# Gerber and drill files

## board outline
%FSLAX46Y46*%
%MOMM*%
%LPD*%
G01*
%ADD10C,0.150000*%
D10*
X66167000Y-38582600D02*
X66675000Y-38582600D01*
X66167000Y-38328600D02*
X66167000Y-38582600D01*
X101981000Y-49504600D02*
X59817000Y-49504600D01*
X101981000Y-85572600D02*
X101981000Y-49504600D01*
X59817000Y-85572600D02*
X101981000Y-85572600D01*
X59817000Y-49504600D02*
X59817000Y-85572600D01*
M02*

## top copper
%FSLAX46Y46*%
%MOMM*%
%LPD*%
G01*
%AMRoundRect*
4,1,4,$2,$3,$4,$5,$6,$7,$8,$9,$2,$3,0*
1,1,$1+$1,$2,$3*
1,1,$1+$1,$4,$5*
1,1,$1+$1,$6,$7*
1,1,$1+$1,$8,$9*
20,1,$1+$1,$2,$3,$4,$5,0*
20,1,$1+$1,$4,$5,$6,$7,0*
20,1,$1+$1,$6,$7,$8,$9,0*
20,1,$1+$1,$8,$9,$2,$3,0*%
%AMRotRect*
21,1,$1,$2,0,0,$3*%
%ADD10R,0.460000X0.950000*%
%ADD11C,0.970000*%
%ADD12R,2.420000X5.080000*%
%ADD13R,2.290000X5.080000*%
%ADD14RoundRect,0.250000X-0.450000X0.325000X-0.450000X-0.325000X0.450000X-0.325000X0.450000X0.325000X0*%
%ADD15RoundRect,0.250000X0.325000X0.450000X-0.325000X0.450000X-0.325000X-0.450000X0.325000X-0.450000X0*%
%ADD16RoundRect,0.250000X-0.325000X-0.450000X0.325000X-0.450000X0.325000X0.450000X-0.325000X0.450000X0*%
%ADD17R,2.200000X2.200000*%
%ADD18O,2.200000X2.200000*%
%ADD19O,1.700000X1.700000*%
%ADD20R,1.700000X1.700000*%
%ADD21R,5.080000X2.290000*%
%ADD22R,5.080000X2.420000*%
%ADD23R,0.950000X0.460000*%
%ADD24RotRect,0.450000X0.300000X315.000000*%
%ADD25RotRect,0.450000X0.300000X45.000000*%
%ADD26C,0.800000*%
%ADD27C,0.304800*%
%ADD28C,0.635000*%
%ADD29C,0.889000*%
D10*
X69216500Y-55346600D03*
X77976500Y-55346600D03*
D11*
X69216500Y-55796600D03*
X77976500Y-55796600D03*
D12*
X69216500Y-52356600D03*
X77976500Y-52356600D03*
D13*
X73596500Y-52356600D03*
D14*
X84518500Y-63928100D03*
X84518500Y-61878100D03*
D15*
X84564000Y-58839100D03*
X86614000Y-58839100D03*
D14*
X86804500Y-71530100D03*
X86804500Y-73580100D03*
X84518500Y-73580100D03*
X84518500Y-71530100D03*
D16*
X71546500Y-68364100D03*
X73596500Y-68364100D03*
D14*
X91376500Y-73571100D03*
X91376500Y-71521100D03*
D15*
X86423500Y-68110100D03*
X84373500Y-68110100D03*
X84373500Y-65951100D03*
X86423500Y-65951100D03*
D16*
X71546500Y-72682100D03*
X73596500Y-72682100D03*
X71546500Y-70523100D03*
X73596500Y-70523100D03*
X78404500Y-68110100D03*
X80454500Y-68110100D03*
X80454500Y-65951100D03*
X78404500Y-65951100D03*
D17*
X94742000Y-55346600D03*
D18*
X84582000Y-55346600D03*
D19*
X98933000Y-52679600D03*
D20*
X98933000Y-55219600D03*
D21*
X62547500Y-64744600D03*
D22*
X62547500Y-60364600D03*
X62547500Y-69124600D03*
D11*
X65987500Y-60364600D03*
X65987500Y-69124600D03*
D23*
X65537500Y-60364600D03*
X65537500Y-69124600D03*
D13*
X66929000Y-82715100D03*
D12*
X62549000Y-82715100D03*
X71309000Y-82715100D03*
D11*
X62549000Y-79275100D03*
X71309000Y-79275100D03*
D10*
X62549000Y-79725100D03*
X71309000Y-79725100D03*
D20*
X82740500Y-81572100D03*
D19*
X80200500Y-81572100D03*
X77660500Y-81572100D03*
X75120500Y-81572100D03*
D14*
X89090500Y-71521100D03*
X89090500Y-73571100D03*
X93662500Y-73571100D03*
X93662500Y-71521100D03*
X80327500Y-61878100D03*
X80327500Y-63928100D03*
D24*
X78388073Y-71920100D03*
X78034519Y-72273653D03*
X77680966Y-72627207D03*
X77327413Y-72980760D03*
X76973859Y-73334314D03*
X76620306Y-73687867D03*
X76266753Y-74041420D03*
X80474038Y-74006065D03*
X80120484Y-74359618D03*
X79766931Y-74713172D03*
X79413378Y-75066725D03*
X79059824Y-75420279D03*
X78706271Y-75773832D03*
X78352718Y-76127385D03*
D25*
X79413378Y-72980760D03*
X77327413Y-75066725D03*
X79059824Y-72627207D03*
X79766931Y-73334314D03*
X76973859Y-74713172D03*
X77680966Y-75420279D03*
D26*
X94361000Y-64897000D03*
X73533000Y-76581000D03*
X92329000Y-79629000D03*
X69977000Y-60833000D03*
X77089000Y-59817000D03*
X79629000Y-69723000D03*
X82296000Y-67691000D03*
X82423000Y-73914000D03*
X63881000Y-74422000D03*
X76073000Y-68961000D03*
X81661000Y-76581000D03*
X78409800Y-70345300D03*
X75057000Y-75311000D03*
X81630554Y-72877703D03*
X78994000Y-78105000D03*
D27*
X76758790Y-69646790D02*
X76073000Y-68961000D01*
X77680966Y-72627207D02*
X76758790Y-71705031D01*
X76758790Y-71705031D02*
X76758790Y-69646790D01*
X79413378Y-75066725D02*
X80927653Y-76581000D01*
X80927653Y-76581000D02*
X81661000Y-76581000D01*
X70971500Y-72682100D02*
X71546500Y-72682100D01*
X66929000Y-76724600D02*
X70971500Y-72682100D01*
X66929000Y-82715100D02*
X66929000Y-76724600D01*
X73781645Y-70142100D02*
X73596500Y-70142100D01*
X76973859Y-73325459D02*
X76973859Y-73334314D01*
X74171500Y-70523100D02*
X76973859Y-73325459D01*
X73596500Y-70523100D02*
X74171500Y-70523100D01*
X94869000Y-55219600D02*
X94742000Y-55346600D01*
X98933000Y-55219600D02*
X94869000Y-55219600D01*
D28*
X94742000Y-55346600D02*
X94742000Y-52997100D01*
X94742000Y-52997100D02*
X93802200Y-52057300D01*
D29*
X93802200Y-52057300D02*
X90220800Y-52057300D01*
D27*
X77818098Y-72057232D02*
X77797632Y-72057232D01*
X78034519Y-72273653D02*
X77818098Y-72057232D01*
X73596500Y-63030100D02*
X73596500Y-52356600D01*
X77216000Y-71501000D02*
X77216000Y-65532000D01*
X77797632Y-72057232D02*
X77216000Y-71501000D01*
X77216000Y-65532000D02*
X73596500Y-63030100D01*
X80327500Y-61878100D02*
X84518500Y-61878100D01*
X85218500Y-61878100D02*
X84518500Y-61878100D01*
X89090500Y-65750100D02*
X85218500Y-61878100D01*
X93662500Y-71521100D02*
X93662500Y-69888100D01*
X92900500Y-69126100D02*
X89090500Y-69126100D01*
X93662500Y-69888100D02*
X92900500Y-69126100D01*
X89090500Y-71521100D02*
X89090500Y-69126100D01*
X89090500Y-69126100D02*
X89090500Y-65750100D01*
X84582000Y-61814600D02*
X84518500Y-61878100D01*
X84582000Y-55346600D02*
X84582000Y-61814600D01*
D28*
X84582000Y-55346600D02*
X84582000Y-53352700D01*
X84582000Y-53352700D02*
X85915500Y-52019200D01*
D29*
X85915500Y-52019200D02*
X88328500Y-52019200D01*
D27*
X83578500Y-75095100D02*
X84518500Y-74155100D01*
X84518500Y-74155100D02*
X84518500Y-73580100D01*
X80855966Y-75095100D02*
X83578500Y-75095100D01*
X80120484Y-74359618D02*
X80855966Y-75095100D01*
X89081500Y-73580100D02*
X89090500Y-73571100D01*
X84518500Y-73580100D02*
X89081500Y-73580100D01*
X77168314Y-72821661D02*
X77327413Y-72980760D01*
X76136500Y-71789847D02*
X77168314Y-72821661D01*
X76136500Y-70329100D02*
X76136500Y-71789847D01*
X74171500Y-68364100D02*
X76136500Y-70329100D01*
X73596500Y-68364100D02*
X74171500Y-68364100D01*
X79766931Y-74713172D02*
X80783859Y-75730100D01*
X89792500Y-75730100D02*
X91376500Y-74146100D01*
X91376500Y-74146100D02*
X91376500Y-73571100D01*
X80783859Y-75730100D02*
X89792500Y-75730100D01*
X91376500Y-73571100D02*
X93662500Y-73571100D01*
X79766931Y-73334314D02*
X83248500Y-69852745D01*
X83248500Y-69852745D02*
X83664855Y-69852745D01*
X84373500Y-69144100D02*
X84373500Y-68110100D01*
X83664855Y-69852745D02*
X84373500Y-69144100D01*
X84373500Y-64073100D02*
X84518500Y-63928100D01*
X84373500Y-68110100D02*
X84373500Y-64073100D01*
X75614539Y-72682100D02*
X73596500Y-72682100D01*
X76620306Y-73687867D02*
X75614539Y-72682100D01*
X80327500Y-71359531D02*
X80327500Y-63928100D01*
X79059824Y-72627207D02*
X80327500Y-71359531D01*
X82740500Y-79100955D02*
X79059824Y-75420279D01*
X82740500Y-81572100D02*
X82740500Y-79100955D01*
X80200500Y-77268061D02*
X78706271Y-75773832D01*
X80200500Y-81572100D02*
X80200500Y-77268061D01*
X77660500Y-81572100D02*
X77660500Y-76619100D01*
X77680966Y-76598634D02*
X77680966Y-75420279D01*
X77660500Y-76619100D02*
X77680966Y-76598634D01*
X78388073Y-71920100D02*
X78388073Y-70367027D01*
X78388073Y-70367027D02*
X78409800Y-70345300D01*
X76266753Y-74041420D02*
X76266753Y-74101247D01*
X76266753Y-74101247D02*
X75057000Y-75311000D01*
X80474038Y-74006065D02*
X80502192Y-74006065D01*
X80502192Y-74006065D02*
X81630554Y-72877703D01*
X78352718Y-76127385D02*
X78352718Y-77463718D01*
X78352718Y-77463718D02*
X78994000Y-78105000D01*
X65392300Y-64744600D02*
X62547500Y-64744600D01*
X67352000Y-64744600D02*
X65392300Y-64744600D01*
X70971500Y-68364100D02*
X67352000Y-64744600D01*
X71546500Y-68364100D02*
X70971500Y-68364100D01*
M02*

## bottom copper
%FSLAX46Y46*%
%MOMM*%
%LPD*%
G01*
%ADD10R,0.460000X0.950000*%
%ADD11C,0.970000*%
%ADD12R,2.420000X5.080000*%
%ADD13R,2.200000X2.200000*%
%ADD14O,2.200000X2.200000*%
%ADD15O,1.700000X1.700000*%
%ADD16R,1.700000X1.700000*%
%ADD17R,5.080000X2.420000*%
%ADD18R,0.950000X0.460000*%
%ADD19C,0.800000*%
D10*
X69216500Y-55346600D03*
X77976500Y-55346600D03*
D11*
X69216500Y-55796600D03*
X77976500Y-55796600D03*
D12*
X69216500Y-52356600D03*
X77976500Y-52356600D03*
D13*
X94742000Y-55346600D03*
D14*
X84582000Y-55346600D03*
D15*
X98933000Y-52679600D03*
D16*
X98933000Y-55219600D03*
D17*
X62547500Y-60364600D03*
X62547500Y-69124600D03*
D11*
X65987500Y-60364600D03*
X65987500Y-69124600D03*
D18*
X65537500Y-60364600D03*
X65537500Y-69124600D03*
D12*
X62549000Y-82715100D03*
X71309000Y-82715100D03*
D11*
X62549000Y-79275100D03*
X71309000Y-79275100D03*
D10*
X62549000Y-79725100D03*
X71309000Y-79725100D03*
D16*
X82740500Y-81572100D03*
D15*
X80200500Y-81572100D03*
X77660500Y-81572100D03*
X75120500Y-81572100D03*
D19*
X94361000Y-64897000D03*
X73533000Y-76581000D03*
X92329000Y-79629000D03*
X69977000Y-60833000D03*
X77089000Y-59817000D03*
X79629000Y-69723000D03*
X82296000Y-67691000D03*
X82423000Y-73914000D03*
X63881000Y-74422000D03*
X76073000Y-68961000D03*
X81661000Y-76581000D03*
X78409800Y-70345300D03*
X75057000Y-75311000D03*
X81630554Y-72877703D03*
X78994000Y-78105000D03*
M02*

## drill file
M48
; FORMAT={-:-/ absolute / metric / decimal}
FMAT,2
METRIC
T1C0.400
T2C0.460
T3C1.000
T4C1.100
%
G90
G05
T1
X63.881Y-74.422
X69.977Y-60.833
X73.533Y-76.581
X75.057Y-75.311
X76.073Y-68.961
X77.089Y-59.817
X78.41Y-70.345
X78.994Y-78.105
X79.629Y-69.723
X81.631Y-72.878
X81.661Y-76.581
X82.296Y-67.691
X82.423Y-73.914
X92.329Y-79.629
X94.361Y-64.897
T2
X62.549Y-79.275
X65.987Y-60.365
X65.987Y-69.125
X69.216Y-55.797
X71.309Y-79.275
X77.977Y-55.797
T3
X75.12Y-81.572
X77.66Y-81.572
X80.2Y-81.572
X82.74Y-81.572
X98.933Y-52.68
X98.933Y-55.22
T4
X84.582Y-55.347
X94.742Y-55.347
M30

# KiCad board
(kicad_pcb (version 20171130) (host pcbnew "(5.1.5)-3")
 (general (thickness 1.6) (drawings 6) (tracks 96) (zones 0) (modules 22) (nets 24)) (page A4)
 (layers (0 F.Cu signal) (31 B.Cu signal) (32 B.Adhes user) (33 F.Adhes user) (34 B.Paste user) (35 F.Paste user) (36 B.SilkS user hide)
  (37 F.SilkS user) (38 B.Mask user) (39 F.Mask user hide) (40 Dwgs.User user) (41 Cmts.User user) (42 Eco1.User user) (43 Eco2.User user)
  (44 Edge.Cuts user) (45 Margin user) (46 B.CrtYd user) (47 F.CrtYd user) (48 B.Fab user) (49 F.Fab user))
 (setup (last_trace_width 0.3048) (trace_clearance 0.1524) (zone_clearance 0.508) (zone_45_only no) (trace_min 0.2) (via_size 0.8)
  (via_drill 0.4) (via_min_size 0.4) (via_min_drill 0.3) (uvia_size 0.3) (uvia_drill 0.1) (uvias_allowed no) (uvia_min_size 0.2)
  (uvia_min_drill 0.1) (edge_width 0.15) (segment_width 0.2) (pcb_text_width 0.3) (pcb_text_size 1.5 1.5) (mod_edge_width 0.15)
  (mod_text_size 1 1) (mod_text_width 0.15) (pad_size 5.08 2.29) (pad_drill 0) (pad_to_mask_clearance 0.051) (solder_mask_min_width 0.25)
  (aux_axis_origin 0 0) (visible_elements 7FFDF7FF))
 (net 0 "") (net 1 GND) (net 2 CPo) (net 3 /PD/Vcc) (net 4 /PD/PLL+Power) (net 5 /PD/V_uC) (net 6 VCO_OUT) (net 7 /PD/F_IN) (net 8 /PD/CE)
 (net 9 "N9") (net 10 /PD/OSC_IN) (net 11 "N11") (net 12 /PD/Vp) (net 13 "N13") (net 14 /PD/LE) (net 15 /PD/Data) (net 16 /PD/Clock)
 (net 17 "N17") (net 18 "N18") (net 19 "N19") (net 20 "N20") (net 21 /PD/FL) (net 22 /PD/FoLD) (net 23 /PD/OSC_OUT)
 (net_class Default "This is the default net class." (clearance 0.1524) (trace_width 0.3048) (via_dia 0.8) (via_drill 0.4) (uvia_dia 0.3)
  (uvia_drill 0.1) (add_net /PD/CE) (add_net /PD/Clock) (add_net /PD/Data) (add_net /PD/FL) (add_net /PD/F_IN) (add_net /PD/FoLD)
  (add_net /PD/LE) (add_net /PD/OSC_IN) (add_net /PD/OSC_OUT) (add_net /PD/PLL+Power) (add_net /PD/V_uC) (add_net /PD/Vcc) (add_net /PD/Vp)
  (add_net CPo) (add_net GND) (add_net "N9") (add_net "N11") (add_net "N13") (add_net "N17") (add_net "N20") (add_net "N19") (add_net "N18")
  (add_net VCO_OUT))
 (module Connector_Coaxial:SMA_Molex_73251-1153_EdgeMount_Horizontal (layer F.Cu) (at 73.5965 54.0766 270)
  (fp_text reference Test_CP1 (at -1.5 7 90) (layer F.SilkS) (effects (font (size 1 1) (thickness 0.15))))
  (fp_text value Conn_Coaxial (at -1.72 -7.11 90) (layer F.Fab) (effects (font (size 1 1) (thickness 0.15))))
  (pad 2 smd rect (at 1.27 4.38 270) (size 0.95 0.46) (layers B.Cu) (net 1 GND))
  (pad 2 smd rect (at 1.27 -4.38 270) (size 0.95 0.46) (layers B.Cu) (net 1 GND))
  (pad 2 smd rect (at 1.27 4.38 270) (size 0.95 0.46) (layers F.Cu) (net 1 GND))
  (pad 2 smd rect (at 1.27 -4.38 270) (size 0.95 0.46) (layers F.Cu) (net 1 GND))
  (pad 2 thru_hole circle (at 1.72 4.38 270) (size 0.97 0.97) (drill 0.46) (layers *.Cu) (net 1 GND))
  (pad 2 thru_hole circle (at 1.72 -4.38 270) (size 0.97 0.97) (drill 0.46) (layers *.Cu) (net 1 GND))
  (pad 2 smd rect (at -1.72 4.38 270) (size 5.08 2.42) (layers B.Cu B.Paste B.Mask) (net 1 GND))
  (pad 2 smd rect (at -1.72 -4.38 270) (size 5.08 2.42) (layers B.Cu B.Paste B.Mask) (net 1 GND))
  (pad 2 smd rect (at -1.72 4.38 270) (size 5.08 2.42) (layers F.Cu F.Paste F.Mask) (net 1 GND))
  (pad 2 smd rect (at -1.72 -4.38 270) (size 5.08 2.42) (layers F.Cu F.Paste F.Mask) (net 1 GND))
  (pad 1 smd rect (at -1.72 0 270) (size 5.08 2.29) (layers F.Cu F.Paste F.Mask) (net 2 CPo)))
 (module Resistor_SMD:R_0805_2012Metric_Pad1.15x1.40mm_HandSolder (layer F.Cu) (at 84.5185 62.9031 270)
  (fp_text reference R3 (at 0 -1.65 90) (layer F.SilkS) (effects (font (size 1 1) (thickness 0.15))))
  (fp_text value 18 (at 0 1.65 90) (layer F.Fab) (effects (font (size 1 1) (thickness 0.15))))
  (pad 2 smd roundrect (at 1.025 0 270) (size 1.15 1.4) (layers F.Cu F.Paste F.Mask) (roundrect_rratio 0.217391) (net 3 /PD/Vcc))
  (pad 1 smd roundrect (at -1.025 0 270) (size 1.15 1.4) (layers F.Cu F.Paste F.Mask) (roundrect_rratio 0.217391) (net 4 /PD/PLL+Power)))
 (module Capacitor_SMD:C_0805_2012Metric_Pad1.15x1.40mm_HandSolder (layer F.Cu) (at 85.589 58.8391 180)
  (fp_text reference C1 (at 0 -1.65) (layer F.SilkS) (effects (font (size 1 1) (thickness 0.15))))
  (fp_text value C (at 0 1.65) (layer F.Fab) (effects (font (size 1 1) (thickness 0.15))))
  (pad 2 smd roundrect (at 1.025 0 180) (size 1.15 1.4) (layers F.Cu F.Paste F.Mask) (roundrect_rratio 0.217391) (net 4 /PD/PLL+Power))
  (pad 1 smd roundrect (at -1.025 0 180) (size 1.15 1.4) (layers F.Cu F.Paste F.Mask) (roundrect_rratio 0.217391) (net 1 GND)))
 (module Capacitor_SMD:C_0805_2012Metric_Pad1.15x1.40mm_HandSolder (layer F.Cu) (at 86.8045 72.5551 270)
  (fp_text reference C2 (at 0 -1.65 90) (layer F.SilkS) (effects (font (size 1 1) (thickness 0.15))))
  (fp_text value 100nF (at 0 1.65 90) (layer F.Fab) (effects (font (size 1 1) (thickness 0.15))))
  (pad 1 smd roundrect (at -1.025 0 270) (size 1.15 1.4) (layers F.Cu F.Paste F.Mask) (roundrect_rratio 0.217391) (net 1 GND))
  (pad 2 smd roundrect (at 1.025 0 270) (size 1.15 1.4) (layers F.Cu F.Paste F.Mask) (roundrect_rratio 0.217391) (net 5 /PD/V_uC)))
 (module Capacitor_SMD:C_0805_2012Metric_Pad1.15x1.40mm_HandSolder (layer F.Cu) (at 84.5185 72.5551 270)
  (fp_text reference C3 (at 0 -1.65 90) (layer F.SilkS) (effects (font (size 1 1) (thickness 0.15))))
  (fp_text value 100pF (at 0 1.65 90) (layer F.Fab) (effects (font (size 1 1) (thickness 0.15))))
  (pad 2 smd roundrect (at 1.025 0 270) (size 1.15 1.4) (layers F.Cu F.Paste F.Mask) (roundrect_rratio 0.217391) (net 5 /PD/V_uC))
  (pad 1 smd roundrect (at -1.025 0 270) (size 1.15 1.4) (layers F.Cu F.Paste F.Mask) (roundrect_rratio 0.217391) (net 1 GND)))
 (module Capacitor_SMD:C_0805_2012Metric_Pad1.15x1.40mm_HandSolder (layer F.Cu) (at 72.5715 68.3641)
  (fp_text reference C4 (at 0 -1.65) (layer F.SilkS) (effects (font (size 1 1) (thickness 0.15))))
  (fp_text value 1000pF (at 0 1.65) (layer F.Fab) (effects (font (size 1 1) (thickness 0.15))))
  (pad 1 smd roundrect (at -1.025 0) (size 1.15 1.4) (layers F.Cu F.Paste F.Mask) (roundrect_rratio 0.217391) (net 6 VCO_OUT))
  (pad 2 smd roundrect (at 1.025 0) (size 1.15 1.4) (layers F.Cu F.Paste F.Mask) (roundrect_rratio 0.217391) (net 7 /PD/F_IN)))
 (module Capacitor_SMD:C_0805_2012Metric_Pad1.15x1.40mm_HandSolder (layer F.Cu) (at 91.3765 72.5461 270)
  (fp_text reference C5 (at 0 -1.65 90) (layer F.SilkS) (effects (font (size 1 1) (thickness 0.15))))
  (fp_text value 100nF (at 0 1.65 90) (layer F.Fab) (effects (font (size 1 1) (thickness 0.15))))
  (pad 2 smd roundrect (at 1.025 0 270) (size 1.15 1.4) (layers F.Cu F.Paste F.Mask) (roundrect_rratio 0.217391) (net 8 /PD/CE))
  (pad 1 smd roundrect (at -1.025 0 270) (size 1.15 1.4) (layers F.Cu F.Paste F.Mask) (roundrect_rratio 0.217391) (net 1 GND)))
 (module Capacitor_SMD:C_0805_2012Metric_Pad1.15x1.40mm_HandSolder (layer F.Cu) (at 85.3985 68.1101 180)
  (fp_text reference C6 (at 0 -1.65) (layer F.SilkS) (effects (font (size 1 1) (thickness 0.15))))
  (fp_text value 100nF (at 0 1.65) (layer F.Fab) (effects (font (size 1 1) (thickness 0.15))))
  (pad 1 smd roundrect (at -1.025 0 180) (size 1.15 1.4) (layers F.Cu F.Paste F.Mask) (roundrect_rratio 0.217391) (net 1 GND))
  (pad 2 smd roundrect (at 1.025 0 180) (size 1.15 1.4) (layers F.Cu F.Paste F.Mask) (roundrect_rratio 0.217391) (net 3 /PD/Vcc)))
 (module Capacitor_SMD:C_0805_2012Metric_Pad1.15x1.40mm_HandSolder (layer F.Cu) (at 85.3985 65.9511 180)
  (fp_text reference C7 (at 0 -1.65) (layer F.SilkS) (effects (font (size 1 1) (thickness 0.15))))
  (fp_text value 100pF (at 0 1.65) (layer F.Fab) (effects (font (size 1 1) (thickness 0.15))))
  (pad 2 smd roundrect (at 1.025 0 180) (size 1.15 1.4) (layers F.Cu F.Paste F.Mask) (roundrect_rratio 0.217391) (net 3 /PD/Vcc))
  (pad 1 smd roundrect (at -1.025 0 180) (size 1.15 1.4) (layers F.Cu F.Paste F.Mask) (roundrect_rratio 0.217391) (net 1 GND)))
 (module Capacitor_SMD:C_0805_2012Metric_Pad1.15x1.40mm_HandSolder (layer F.Cu) (at 72.5715 72.6821)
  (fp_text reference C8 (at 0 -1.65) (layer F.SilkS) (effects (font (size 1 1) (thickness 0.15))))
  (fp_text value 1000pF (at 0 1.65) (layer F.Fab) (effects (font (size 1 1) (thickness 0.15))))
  (pad 1 smd roundrect (at -1.025 0) (size 1.15 1.4) (layers F.Cu F.Paste F.Mask) (roundrect_rratio 0.217391) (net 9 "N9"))
  (pad 2 smd roundrect (at 1.025 0) (size 1.15 1.4) (layers F.Cu F.Paste F.Mask) (roundrect_rratio 0.217391) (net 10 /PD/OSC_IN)))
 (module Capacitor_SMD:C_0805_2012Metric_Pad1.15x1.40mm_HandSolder (layer F.Cu) (at 72.5715 70.5231)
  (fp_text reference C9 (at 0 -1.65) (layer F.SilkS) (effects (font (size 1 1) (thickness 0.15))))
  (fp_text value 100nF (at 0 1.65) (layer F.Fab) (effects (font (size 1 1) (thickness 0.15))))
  (pad 1 smd roundrect (at -1.025 0) (size 1.15 1.4) (layers F.Cu F.Paste F.Mask) (roundrect_rratio 0.217391) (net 1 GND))
  (pad 2 smd roundrect (at 1.025 0) (size 1.15 1.4) (layers F.Cu F.Paste F.Mask) (roundrect_rratio 0.217391) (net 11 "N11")))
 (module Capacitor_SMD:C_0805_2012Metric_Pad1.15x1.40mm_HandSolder (layer F.Cu) (at 79.4295 68.1101)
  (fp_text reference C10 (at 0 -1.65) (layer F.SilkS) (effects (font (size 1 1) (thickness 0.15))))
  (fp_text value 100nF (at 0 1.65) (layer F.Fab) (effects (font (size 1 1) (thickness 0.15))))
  (pad 1 smd roundrect (at -1.025 0) (size 1.15 1.4) (layers F.Cu F.Paste F.Mask) (roundrect_rratio 0.217391) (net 1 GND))
  (pad 2 smd roundrect (at 1.025 0) (size 1.15 1.4) (layers F.Cu F.Paste F.Mask) (roundrect_rratio 0.217391) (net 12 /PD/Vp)))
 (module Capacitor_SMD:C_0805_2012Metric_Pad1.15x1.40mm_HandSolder (layer F.Cu) (at 79.4295 65.9511)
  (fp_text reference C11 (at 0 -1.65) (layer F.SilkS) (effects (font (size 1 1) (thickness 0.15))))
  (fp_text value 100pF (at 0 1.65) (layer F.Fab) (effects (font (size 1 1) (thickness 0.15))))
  (pad 2 smd roundrect (at 1.025 0) (size 1.15 1.4) (layers F.Cu F.Paste F.Mask) (roundrect_rratio 0.217391) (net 12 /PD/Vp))
  (pad 1 smd roundrect (at -1.025 0) (size 1.15 1.4) (layers F.Cu F.Paste F.Mask) (roundrect_rratio 0.217391) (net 1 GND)))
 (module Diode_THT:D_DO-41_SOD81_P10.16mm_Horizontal (layer F.Cu) (at 94.742 55.3466 180)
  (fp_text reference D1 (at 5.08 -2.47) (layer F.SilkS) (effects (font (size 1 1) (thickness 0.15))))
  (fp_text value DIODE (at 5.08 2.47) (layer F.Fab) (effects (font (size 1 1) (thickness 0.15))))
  (pad 1 thru_hole rect (at 0 0 180) (size 2.2 2.2) (drill 1.1) (layers *.Cu *.Mask) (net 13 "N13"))
  (pad 2 thru_hole oval (at 10.16 0 180) (size 2.2 2.2) (drill 1.1) (layers *.Cu *.Mask) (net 4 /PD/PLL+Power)))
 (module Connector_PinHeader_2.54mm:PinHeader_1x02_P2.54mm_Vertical (layer F.Cu) (at 98.933 55.2196 180)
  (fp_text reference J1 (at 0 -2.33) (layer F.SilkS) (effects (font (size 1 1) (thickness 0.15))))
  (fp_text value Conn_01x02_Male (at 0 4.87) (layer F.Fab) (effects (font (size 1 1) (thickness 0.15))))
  (pad 2 thru_hole oval (at 0 2.54 180) (size 1.7 1.7) (drill 1) (layers *.Cu *.Mask) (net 1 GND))
  (pad 1 thru_hole rect (at 0 0 180) (size 1.7 1.7) (drill 1) (layers *.Cu *.Mask) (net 13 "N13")))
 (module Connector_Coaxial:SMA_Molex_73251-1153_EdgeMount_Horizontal (layer F.Cu) (at 64.2675 64.7446)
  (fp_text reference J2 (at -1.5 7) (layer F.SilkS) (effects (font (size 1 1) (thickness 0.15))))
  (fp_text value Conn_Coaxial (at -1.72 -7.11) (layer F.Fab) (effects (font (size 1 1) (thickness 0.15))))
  (pad 1 smd rect (at -1.72 0) (size 5.08 2.29) (layers F.Cu F.Paste F.Mask) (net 6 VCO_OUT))
  (pad 2 smd rect (at -1.72 -4.38) (size 5.08 2.42) (layers F.Cu F.Paste F.Mask) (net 1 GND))
  (pad 2 smd rect (at -1.72 4.38) (size 5.08 2.42) (layers F.Cu F.Paste F.Mask) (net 1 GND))
  (pad 2 smd rect (at -1.72 -4.38) (size 5.08 2.42) (layers B.Cu B.Paste B.Mask) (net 1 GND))
  (pad 2 smd rect (at -1.72 4.38) (size 5.08 2.42) (layers B.Cu B.Paste B.Mask) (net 1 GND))
  (pad 2 thru_hole circle (at 1.72 -4.38) (size 0.97 0.97) (drill 0.46) (layers *.Cu) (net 1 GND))
  (pad 2 thru_hole circle (at 1.72 4.38) (size 0.97 0.97) (drill 0.46) (layers *.Cu) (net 1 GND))
  (pad 2 smd rect (at 1.27 -4.38) (size 0.95 0.46) (layers F.Cu) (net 1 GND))
  (pad 2 smd rect (at 1.27 4.38) (size 0.95 0.46) (layers F.Cu) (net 1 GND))
  (pad 2 smd rect (at 1.27 -4.38) (size 0.95 0.46) (layers B.Cu) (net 1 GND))
  (pad 2 smd rect (at 1.27 4.38) (size 0.95 0.46) (layers B.Cu) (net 1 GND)))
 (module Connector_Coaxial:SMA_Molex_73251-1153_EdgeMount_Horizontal (layer F.Cu) (at 66.929 80.9951 90)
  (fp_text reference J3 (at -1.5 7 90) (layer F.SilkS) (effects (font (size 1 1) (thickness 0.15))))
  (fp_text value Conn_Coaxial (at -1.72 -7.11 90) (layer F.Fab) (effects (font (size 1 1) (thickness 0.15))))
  (pad 1 smd rect (at -1.72 0 90) (size 5.08 2.29) (layers F.Cu F.Paste F.Mask) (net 9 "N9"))
  (pad 2 smd rect (at -1.72 -4.38 90) (size 5.08 2.42) (layers F.Cu F.Paste F.Mask) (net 1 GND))
  (pad 2 smd rect (at -1.72 4.38 90) (size 5.08 2.42) (layers F.Cu F.Paste F.Mask) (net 1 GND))
  (pad 2 smd rect (at -1.72 -4.38 90) (size 5.08 2.42) (layers B.Cu B.Paste B.Mask) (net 1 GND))
  (pad 2 smd rect (at -1.72 4.38 90) (size 5.08 2.42) (layers B.Cu B.Paste B.Mask) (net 1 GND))
  (pad 2 thru_hole circle (at 1.72 -4.38 90) (size 0.97 0.97) (drill 0.46) (layers *.Cu) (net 1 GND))
  (pad 2 thru_hole circle (at 1.72 4.38 90) (size 0.97 0.97) (drill 0.46) (layers *.Cu) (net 1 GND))
  (pad 2 smd rect (at 1.27 -4.38 90) (size 0.95 0.46) (layers F.Cu) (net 1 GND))
  (pad 2 smd rect (at 1.27 4.38 90) (size 0.95 0.46) (layers F.Cu) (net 1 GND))
  (pad 2 smd rect (at 1.27 -4.38 90) (size 0.95 0.46) (layers B.Cu) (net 1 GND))
  (pad 2 smd rect (at 1.27 4.38 90) (size 0.95 0.46) (layers B.Cu) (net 1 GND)))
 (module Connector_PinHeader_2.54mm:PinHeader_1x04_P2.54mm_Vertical (layer F.Cu) (at 82.7405 81.5721 270)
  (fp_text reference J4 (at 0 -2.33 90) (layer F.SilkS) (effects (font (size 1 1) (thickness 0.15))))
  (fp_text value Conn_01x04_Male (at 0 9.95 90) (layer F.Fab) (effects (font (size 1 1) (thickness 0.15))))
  (pad 1 thru_hole rect (at 0 0 270) (size 1.7 1.7) (drill 1) (layers *.Cu *.Mask) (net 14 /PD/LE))
  (pad 2 thru_hole oval (at 0 2.54 270) (size 1.7 1.7) (drill 1) (layers *.Cu *.Mask) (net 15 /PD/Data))
  (pad 3 thru_hole oval (at 0 5.08 270) (size 1.7 1.7) (drill 1) (layers *.Cu *.Mask) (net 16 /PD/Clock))
  (pad 4 thru_hole oval (at 0 7.62 270) (size 1.7 1.7) (drill 1) (layers *.Cu *.Mask) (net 1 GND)))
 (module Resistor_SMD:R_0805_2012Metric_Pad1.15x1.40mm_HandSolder (layer F.Cu) (at 89.0905 72.5461 270)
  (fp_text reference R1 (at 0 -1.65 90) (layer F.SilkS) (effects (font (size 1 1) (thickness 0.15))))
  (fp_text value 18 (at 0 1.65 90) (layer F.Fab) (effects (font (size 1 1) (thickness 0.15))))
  (pad 1 smd roundrect (at -1.025 0 270) (size 1.15 1.4) (layers F.Cu F.Paste F.Mask) (roundrect_rratio 0.217391) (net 4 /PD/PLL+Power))
  (pad 2 smd roundrect (at 1.025 0 270) (size 1.15 1.4) (layers F.Cu F.Paste F.Mask) (roundrect_rratio 0.217391) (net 5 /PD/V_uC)))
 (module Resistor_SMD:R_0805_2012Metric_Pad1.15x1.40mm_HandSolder (layer F.Cu) (at 93.6625 72.5461 270)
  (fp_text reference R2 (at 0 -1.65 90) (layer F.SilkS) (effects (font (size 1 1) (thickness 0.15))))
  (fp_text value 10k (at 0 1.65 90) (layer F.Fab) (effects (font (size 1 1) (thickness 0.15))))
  (pad 2 smd roundrect (at 1.025 0 270) (size 1.15 1.4) (layers F.Cu F.Paste F.Mask) (roundrect_rratio 0.217391) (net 8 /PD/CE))
  (pad 1 smd roundrect (at -1.025 0 270) (size 1.15 1.4) (layers F.Cu F.Paste F.Mask) (roundrect_rratio 0.217391) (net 4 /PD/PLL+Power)))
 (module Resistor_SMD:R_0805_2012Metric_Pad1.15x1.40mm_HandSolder (layer F.Cu) (at 80.3275 62.9031 270)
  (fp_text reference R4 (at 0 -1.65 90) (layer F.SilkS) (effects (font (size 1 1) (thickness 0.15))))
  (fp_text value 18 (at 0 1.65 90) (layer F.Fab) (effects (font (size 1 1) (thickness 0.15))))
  (pad 1 smd roundrect (at -1.025 0 270) (size 1.15 1.4) (layers F.Cu F.Paste F.Mask) (roundrect_rratio 0.217391) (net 4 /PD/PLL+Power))
  (pad 2 smd roundrect (at 1.025 0 270) (size 1.15 1.4) (layers F.Cu F.Paste F.Mask) (roundrect_rratio 0.217391) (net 12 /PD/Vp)))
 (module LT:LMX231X (layer F.Cu) (at 81.2165 71.9201 315)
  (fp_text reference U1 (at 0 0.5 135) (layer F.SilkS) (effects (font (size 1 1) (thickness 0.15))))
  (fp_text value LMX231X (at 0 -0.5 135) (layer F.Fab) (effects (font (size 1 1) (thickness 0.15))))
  (pad 1 smd rect (at -2 2 315) (size 0.45 0.3) (layers F.Cu F.Paste F.Mask) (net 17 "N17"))
  (pad 2 smd rect (at -2 2.5 315) (size 0.45 0.3) (layers F.Cu F.Paste F.Mask) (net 2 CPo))
  (pad 3 smd rect (at -2 3 315) (size 0.45 0.3) (layers F.Cu F.Paste F.Mask) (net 1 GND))
  (pad 4 smd rect (at -2 3.5 315) (size 0.45 0.3) (layers F.Cu F.Paste F.Mask) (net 7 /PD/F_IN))
  (pad 5 smd rect (at -2 4 315) (size 0.45 0.3) (layers F.Cu F.Paste F.Mask) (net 11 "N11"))
  (pad 6 smd rect (at -2 4.5 315) (size 0.45 0.3) (layers F.Cu F.Paste F.Mask) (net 10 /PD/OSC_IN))
  (pad 7 smd rect (at -2 5 315) (size 0.45 0.3) (layers F.Cu F.Paste F.Mask) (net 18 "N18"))
  (pad 17 smd rect (at 0.95 2 315) (size 0.45 0.3) (layers F.Cu F.Paste F.Mask) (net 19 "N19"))
  (pad 16 smd rect (at 0.95 2.5 315) (size 0.45 0.3) (layers F.Cu F.Paste F.Mask) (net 5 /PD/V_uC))
  (pad 15 smd rect (at 0.95 3 315) (size 0.45 0.3) (layers F.Cu F.Paste F.Mask) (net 8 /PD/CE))
  (pad 14 smd rect (at 0.95 3.5 315) (size 0.45 0.3) (layers F.Cu F.Paste F.Mask) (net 1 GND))
  (pad 13 smd rect (at 0.95 4 315) (size 0.45 0.3) (layers F.Cu F.Paste F.Mask) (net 14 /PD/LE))
  (pad 12 smd rect (at 0.95 4.5 315) (size 0.45 0.3) (layers F.Cu F.Paste F.Mask) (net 15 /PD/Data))
  (pad 11 smd rect (at 0.95 5 315) (size 0.45 0.3) (layers F.Cu F.Paste F.Mask) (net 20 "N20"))
  (pad 19 smd rect (at -0.525 2.025 45) (size 0.45 0.3) (layers F.Cu F.Paste F.Mask) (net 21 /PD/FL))
  (pad 9 smd rect (at -0.525 4.975 45) (size 0.45 0.3) (layers F.Cu F.Paste F.Mask) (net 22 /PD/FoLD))
  (pad 20 smd rect (at -1.025 2.025 45) (size 0.45 0.3) (layers F.Cu F.Paste F.Mask) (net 12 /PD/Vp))
  (pad 18 smd rect (at -0.025 2.025 45) (size 0.45 0.3) (layers F.Cu F.Paste F.Mask) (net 3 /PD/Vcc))
  (pad 8 smd rect (at -1.025 4.975 45) (size 0.45 0.3) (layers F.Cu F.Paste F.Mask) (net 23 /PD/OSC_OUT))
  (pad 10 smd rect (at -0.025 4.975 45) (size 0.45 0.3) (layers F.Cu F.Paste F.Mask) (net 16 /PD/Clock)))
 (gr_line (start 66.167 38.5826) (end 66.675 38.5826) (layer Edge.Cuts) (width 0.15))
 (gr_line (start 66.167 38.3286) (end 66.167 38.5826) (layer Edge.Cuts) (width 0.15))
 (gr_line (start 101.981 49.5046) (end 59.817 49.5046) (layer Edge.Cuts) (width 0.15))
 (gr_line (start 101.981 85.5726) (end 101.981 49.5046) (layer Edge.Cuts) (width 0.15))
 (gr_line (start 59.817 85.5726) (end 101.981 85.5726) (layer Edge.Cuts) (width 0.15))
 (gr_line (start 59.817 49.5046) (end 59.817 85.5726) (layer Edge.Cuts) (width 0.15))
 (via (at 94.361 64.897) (size 0.8) (drill 0.4) (layers F.Cu B.Cu) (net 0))
 (via (at 73.533 76.581) (size 0.8) (drill 0.4) (layers F.Cu B.Cu) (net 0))
 (via (at 92.329 79.629) (size 0.8) (drill 0.4) (layers F.Cu B.Cu) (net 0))
 (via (at 69.977 60.833) (size 0.8) (drill 0.4) (layers F.Cu B.Cu) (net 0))
 (via (at 77.089 59.817) (size 0.8) (drill 0.4) (layers F.Cu B.Cu) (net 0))
 (via (at 79.629 69.723) (size 0.8) (drill 0.4) (layers F.Cu B.Cu) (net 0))
 (via (at 82.296 67.691) (size 0.8) (drill 0.4) (layers F.Cu B.Cu) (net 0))
 (via (at 82.423 73.914) (size 0.8) (drill 0.4) (layers F.Cu B.Cu) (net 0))
 (via (at 63.881 74.422) (size 0.8) (drill 0.4) (layers F.Cu B.Cu) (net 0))
 (via (at 76.073 68.961) (size 0.8) (drill 0.4) (layers F.Cu B.Cu) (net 1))
 (segment (start 76.75879 69.64679) (end 76.073 68.961) (width 0.3048) (layer F.Cu) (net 1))
 (segment (start 77.680966 72.627207) (end 76.75879 71.705031) (width 0.3048) (layer F.Cu) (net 1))
 (segment (start 76.75879 71.705031) (end 76.75879 69.64679) (width 0.3048) (layer F.Cu) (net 1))
 (via (at 81.661 76.581) (size 0.8) (drill 0.4) (layers F.Cu B.Cu) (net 1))
 (segment (start 79.413378 75.066725) (end 80.927653 76.581) (width 0.3048) (layer F.Cu) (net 1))
 (segment (start 80.927653 76.581) (end 81.661 76.581) (width 0.3048) (layer F.Cu) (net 1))
 (segment (start 70.9715 72.6821) (end 71.5465 72.6821) (width 0.3048) (layer F.Cu) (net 9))
 (segment (start 66.929 76.7246) (end 70.9715 72.6821) (width 0.3048) (layer F.Cu) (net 9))
 (segment (start 66.929 82.7151) (end 66.929 76.7246) (width 0.3048) (layer F.Cu) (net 9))
 (segment (start 73.781645 70.1421) (end 73.5965 70.1421) (width 0.3048) (layer F.Cu) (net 11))
 (segment (start 76.973859 73.325459) (end 76.973859 73.334314) (width 0.3048) (layer F.Cu) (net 11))
 (segment (start 74.1715 70.5231) (end 76.973859 73.325459) (width 0.3048) (layer F.Cu) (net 11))
 (segment (start 73.5965 70.5231) (end 74.1715 70.5231) (width 0.3048) (layer F.Cu) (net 11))
 (segment (start 94.869 55.2196) (end 94.742 55.3466) (width 0.3048) (layer F.Cu) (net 13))
 (segment (start 98.933 55.2196) (end 94.869 55.2196) (width 0.3048) (layer F.Cu) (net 13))
 (segment (start 94.742 55.3466) (end 94.742 52.9971) (width 0.635) (layer F.Cu) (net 13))
 (segment (start 94.742 52.9971) (end 93.8022 52.0573) (width 0.635) (layer F.Cu) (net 13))
 (segment (start 93.8022 52.0573) (end 90.2208 52.0573) (width 0.889) (layer F.Cu) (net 13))
 (segment (start 77.818098 72.057232) (end 77.797632 72.057232) (width 0.3048) (layer F.Cu) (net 2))
 (segment (start 78.034519 72.273653) (end 77.818098 72.057232) (width 0.3048) (layer F.Cu) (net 2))
 (segment (start 73.5965 63.0301) (end 73.5965 52.3566) (width 0.3048) (layer F.Cu) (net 2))
 (segment (start 77.216 71.501) (end 77.216 65.532) (width 0.3048) (layer F.Cu) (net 2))
 (segment (start 77.797632 72.057232) (end 77.216 71.501) (width 0.3048) (layer F.Cu) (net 2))
 (segment (start 77.216 65.532) (end 73.5965 63.0301) (width 0.3048) (layer F.Cu) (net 2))
 (segment (start 80.3275 61.8781) (end 84.5185 61.8781) (width 0.3048) (layer F.Cu) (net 4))
 (segment (start 85.2185 61.8781) (end 84.5185 61.8781) (width 0.3048) (layer F.Cu) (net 4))
 (segment (start 89.0905 65.7501) (end 85.2185 61.8781) (width 0.3048) (layer F.Cu) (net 4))
 (segment (start 93.6625 71.5211) (end 93.6625 69.8881) (width 0.3048) (layer F.Cu) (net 4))
 (segment (start 92.9005 69.1261) (end 89.0905 69.1261) (width 0.3048) (layer F.Cu) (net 4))
 (segment (start 93.6625 69.8881) (end 92.9005 69.1261) (width 0.3048) (layer F.Cu) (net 4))
 (segment (start 89.0905 71.5211) (end 89.0905 69.1261) (width 0.3048) (layer F.Cu) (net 4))
 (segment (start 89.0905 69.1261) (end 89.0905 65.7501) (width 0.3048) (layer F.Cu) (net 4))
 (segment (start 84.582 61.8146) (end 84.5185 61.8781) (width 0.3048) (layer F.Cu) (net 4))
 (segment (start 84.582 55.3466) (end 84.582 61.8146) (width 0.3048) (layer F.Cu) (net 4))
 (segment (start 84.582 55.3466) (end 84.582 53.3527) (width 0.635) (layer F.Cu) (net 4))
 (segment (start 84.582 53.3527) (end 85.9155 52.0192) (width 0.635) (layer F.Cu) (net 4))
 (segment (start 85.9155 52.0192) (end 88.3285 52.0192) (width 0.889) (layer F.Cu) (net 4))
 (segment (start 83.5785 75.0951) (end 84.5185 74.1551) (width 0.3048) (layer F.Cu) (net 5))
 (segment (start 84.5185 74.1551) (end 84.5185 73.5801) (width 0.3048) (layer F.Cu) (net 5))
 (segment (start 80.855966 75.0951) (end 83.5785 75.0951) (width 0.3048) (layer F.Cu) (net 5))
 (segment (start 80.120484 74.359618) (end 80.855966 75.0951) (width 0.3048) (layer F.Cu) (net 5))
 (segment (start 89.0815 73.5801) (end 89.0905 73.5711) (width 0.3048) (layer F.Cu) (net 5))
 (segment (start 84.5185 73.5801) (end 89.0815 73.5801) (width 0.3048) (layer F.Cu) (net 5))
 (segment (start 77.168314 72.821661) (end 77.327413 72.98076) (width 0.3048) (layer F.Cu) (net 7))
 (segment (start 76.1365 71.789847) (end 77.168314 72.821661) (width 0.3048) (layer F.Cu) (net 7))
 (segment (start 76.1365 70.3291) (end 76.1365 71.789847) (width 0.3048) (layer F.Cu) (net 7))
 (segment (start 74.1715 68.3641) (end 76.1365 70.3291) (width 0.3048) (layer F.Cu) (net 7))
 (segment (start 73.5965 68.3641) (end 74.1715 68.3641) (width 0.3048) (layer F.Cu) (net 7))
 (segment (start 79.766931 74.713172) (end 80.783859 75.7301) (width 0.3048) (layer F.Cu) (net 8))
 (segment (start 89.7925 75.7301) (end 91.3765 74.1461) (width 0.3048) (layer F.Cu) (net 8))
 (segment (start 91.3765 74.1461) (end 91.3765 73.5711) (width 0.3048) (layer F.Cu) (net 8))
 (segment (start 80.783859 75.7301) (end 89.7925 75.7301) (width 0.3048) (layer F.Cu) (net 8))
 (segment (start 91.3765 73.5711) (end 93.6625 73.5711) (width 0.3048) (layer F.Cu) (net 8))
 (segment (start 79.766931 73.334314) (end 83.2485 69.852745) (width 0.3048) (layer F.Cu) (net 3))
 (segment (start 83.2485 69.852745) (end 83.664855 69.852745) (width 0.3048) (layer F.Cu) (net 3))
 (segment (start 84.3735 69.1441) (end 84.3735 68.1101) (width 0.3048) (layer F.Cu) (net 3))
 (segment (start 83.664855 69.852745) (end 84.3735 69.1441) (width 0.3048) (layer F.Cu) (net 3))
 (segment (start 84.3735 64.0731) (end 84.5185 63.9281) (width 0.3048) (layer F.Cu) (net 3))
 (segment (start 84.3735 68.1101) (end 84.3735 64.0731) (width 0.3048) (layer F.Cu) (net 3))
 (segment (start 75.614539 72.6821) (end 73.5965 72.6821) (width 0.3048) (layer F.Cu) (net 10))
 (segment (start 76.620306 73.687867) (end 75.614539 72.6821) (width 0.3048) (layer F.Cu) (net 10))
 (segment (start 80.3275 71.359531) (end 80.3275 63.9281) (width 0.3048) (layer F.Cu) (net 12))
 (segment (start 79.059824 72.627207) (end 80.3275 71.359531) (width 0.3048) (layer F.Cu) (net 12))
 (segment (start 82.7405 79.100955) (end 79.059824 75.420279) (width 0.3048) (layer F.Cu) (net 14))
 (segment (start 82.7405 81.5721) (end 82.7405 79.100955) (width 0.3048) (layer F.Cu) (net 14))
 (segment (start 80.2005 77.268061) (end 78.706271 75.773832) (width 0.3048) (layer F.Cu) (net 15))
 (segment (start 80.2005 81.5721) (end 80.2005 77.268061) (width 0.3048) (layer F.Cu) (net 15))
 (segment (start 77.6605 81.5721) (end 77.6605 76.6191) (width 0.3048) (layer F.Cu) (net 16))
 (segment (start 77.680966 76.598634) (end 77.680966 75.420279) (width 0.3048) (layer F.Cu) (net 16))
 (segment (start 77.6605 76.6191) (end 77.680966 76.598634) (width 0.3048) (layer F.Cu) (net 16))
 (via (at 78.4098 70.3453) (size 0.8) (drill 0.4) (layers F.Cu B.Cu) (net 17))
 (segment (start 78.388073 71.9201) (end 78.388073 70.367027) (width 0.3048) (layer F.Cu) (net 17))
 (segment (start 78.388073 70.367027) (end 78.4098 70.3453) (width 0.3048) (layer F.Cu) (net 17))
 (via (at 75.057 75.311) (size 0.8) (drill 0.4) (layers F.Cu B.Cu) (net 18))
 (segment (start 76.266753 74.04142) (end 76.266753 74.101247) (width 0.3048) (layer F.Cu) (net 18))
 (segment (start 76.266753 74.101247) (end 75.057 75.311) (width 0.3048) (layer F.Cu) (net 18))
 (via (at 81.630554 72.877703) (size 0.8) (drill 0.4) (layers F.Cu B.Cu) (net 19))
 (segment (start 80.474038 74.006065) (end 80.502192 74.006065) (width 0.3048) (layer F.Cu) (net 19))
 (segment (start 80.502192 74.006065) (end 81.630554 72.877703) (width 0.3048) (layer F.Cu) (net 19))
 (via (at 78.994 78.105) (size 0.8) (drill 0.4) (layers F.Cu B.Cu) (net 20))
 (segment (start 78.352718 76.127385) (end 78.352718 77.463718) (width 0.3048) (layer F.Cu) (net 20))
 (segment (start 78.352718 77.463718) (end 78.994 78.105) (width 0.3048) (layer F.Cu) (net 20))
 (segment (start 65.3923 64.7446) (end 62.5475 64.7446) (width 0.3048) (layer F.Cu) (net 6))
 (segment (start 67.352 64.7446) (end 65.3923 64.7446) (width 0.3048) (layer F.Cu) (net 6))
 (segment (start 70.9715 68.3641) (end 67.352 64.7446) (width 0.3048) (layer F.Cu) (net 6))
 (segment (start 71.5465 68.3641) (end 70.9715 68.3641) (width 0.3048) (layer F.Cu) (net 6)))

